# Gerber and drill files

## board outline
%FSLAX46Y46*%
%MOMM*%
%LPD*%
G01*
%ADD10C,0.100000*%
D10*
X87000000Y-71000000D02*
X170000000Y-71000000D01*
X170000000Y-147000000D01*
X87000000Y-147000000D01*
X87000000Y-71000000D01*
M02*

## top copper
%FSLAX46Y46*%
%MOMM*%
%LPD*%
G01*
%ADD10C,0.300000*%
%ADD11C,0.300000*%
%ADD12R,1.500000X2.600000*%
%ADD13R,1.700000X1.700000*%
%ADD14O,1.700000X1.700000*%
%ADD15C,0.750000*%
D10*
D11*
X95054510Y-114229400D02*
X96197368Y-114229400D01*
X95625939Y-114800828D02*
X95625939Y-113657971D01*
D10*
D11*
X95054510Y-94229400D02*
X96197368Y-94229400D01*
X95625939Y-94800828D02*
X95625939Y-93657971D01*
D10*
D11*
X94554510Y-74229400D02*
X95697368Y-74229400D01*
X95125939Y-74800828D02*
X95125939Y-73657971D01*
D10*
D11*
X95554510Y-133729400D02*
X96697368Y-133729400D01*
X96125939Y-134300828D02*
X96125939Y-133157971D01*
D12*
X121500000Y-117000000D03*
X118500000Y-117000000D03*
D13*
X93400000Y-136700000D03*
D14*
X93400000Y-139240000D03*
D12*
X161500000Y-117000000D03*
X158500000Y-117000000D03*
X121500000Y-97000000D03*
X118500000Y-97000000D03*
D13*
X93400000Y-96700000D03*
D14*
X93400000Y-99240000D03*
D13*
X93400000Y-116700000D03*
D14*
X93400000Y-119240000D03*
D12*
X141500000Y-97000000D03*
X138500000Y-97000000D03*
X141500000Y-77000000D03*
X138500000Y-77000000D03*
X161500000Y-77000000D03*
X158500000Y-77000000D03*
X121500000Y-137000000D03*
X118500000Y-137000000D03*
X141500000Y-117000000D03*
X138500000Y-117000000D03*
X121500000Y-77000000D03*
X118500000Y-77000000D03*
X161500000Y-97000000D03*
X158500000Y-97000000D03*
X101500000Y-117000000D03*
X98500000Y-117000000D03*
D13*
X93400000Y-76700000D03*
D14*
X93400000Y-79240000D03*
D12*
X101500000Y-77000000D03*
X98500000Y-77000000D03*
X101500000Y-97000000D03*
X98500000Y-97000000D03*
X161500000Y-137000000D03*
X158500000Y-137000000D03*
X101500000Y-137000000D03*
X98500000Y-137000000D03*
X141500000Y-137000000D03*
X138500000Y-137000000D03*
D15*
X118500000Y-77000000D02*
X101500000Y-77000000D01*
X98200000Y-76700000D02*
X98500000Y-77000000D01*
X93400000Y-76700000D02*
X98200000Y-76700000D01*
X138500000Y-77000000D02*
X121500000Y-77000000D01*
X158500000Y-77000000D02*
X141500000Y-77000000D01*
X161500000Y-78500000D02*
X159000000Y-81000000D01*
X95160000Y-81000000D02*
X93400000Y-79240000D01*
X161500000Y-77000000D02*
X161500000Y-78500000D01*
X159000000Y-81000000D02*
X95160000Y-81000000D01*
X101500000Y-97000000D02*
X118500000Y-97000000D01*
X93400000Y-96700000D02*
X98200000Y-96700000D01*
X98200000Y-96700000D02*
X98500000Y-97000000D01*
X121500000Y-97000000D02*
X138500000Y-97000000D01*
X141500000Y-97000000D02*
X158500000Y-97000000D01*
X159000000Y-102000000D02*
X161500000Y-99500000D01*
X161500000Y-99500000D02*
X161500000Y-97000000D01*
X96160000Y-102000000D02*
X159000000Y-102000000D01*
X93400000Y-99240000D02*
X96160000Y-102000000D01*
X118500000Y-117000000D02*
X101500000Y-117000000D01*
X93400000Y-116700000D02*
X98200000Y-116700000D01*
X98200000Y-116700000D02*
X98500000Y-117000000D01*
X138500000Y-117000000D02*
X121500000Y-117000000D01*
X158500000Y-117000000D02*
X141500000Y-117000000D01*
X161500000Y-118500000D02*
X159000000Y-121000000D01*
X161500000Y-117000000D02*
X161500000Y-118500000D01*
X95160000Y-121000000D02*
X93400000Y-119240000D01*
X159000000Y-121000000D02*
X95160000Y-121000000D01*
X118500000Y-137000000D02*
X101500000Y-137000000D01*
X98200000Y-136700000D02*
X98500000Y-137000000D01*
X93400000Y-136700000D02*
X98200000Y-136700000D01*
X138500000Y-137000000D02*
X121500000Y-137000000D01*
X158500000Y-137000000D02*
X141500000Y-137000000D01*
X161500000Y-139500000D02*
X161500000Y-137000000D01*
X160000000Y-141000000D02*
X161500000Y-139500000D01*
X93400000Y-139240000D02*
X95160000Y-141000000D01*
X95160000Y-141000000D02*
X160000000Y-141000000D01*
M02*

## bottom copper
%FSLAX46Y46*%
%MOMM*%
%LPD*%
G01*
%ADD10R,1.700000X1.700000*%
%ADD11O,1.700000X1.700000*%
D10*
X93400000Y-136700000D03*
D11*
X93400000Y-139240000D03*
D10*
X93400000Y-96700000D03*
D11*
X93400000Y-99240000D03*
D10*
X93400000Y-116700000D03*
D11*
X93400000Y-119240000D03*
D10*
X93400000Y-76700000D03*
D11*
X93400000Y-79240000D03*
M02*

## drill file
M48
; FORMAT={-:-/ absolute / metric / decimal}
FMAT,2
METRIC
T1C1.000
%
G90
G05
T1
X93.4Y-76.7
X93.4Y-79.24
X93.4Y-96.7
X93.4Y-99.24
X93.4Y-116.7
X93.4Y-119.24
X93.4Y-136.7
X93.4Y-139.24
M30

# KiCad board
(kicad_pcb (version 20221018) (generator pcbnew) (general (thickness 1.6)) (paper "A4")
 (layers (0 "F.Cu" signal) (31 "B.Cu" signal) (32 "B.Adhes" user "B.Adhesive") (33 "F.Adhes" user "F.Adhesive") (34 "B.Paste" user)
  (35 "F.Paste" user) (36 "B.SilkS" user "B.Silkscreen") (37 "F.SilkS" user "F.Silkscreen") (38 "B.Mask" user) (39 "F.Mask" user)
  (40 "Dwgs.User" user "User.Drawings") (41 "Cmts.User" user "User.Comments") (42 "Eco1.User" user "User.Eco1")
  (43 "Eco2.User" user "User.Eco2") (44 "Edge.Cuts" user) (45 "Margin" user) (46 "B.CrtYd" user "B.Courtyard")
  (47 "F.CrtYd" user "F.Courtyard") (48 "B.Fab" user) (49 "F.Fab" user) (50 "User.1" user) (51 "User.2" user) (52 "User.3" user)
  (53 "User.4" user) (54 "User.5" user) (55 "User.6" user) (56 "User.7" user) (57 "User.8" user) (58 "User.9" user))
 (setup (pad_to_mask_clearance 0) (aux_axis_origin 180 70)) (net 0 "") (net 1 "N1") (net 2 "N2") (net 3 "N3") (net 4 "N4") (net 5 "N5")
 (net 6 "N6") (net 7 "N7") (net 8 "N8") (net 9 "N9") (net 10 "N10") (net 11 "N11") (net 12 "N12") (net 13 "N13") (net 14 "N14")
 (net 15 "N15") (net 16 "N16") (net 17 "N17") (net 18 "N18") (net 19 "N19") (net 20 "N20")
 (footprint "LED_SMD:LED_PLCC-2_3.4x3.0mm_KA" (layer "F.Cu") (at 120 117 180)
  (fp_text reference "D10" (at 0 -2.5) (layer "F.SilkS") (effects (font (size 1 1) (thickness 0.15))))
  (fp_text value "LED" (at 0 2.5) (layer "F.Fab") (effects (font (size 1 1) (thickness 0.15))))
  (pad "1" smd rect (at -1.5 0 180) (size 1.5 2.6) (layers "F.Cu" "F.Paste" "F.Mask") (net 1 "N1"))
  (pad "2" smd rect (at 1.5 0 180) (size 1.5 2.6) (layers "F.Cu" "F.Paste" "F.Mask") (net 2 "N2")))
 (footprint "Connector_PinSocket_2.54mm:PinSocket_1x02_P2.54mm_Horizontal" (layer "F.Cu") (at 93.4 136.7)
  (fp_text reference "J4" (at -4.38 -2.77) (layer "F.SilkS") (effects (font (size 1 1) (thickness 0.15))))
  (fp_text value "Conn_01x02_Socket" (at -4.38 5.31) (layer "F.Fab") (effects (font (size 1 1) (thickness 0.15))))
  (pad "1" thru_hole rect (at 0 0) (size 1.7 1.7) (drill 1) (layers "*.Cu" "*.Mask") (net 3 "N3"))
  (pad "2" thru_hole oval (at 0 2.54) (size 1.7 1.7) (drill 1) (layers "*.Cu" "*.Mask") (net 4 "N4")))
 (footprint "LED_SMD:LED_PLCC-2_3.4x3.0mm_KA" (layer "F.Cu") (at 160 117 180)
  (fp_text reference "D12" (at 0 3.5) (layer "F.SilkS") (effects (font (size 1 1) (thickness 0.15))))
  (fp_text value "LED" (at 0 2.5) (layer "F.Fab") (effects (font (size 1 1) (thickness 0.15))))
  (pad "1" smd rect (at -1.5 0 180) (size 1.5 2.6) (layers "F.Cu" "F.Paste" "F.Mask") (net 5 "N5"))
  (pad "2" smd rect (at 1.5 0 180) (size 1.5 2.6) (layers "F.Cu" "F.Paste" "F.Mask") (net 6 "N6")))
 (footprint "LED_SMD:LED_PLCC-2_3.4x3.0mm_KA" (layer "F.Cu") (at 120 97 180)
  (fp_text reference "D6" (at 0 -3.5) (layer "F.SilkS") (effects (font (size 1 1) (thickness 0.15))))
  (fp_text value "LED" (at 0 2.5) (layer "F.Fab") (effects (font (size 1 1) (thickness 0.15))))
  (pad "1" smd rect (at -1.5 0 180) (size 1.5 2.6) (layers "F.Cu" "F.Paste" "F.Mask") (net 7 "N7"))
  (pad "2" smd rect (at 1.5 0 180) (size 1.5 2.6) (layers "F.Cu" "F.Paste" "F.Mask") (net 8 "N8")))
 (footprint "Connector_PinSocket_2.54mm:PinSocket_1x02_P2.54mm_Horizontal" (layer "F.Cu") (at 93.4 96.7)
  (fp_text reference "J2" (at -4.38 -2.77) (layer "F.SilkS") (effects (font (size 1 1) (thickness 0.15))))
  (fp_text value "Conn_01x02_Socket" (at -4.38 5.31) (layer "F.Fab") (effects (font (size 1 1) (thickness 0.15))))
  (pad "1" thru_hole rect (at 0 0) (size 1.7 1.7) (drill 1) (layers "*.Cu" "*.Mask") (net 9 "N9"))
  (pad "2" thru_hole oval (at 0 2.54) (size 1.7 1.7) (drill 1) (layers "*.Cu" "*.Mask") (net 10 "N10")))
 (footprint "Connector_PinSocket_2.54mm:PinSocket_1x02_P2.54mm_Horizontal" (layer "F.Cu") (at 93.4 116.7)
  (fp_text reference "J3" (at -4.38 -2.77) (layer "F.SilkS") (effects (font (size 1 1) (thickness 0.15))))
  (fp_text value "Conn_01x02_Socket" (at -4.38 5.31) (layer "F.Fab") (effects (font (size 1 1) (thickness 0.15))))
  (pad "1" thru_hole rect (at 0 0) (size 1.7 1.7) (drill 1) (layers "*.Cu" "*.Mask") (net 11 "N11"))
  (pad "2" thru_hole oval (at 0 2.54) (size 1.7 1.7) (drill 1) (layers "*.Cu" "*.Mask") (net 5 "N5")))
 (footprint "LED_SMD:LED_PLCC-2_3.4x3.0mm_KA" (layer "F.Cu") (at 140 97 180)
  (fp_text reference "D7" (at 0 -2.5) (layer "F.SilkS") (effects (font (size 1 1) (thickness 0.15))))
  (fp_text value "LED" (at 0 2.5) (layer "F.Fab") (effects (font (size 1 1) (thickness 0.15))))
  (pad "1" smd rect (at -1.5 0 180) (size 1.5 2.6) (layers "F.Cu" "F.Paste" "F.Mask") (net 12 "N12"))
  (pad "2" smd rect (at 1.5 0 180) (size 1.5 2.6) (layers "F.Cu" "F.Paste" "F.Mask") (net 7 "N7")))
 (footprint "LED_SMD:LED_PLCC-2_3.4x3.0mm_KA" (layer "F.Cu") (at 140 77 180)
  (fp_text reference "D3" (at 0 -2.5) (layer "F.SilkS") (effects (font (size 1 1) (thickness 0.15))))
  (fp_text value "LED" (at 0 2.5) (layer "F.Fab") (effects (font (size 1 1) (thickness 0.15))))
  (pad "1" smd rect (at -1.5 0 180) (size 1.5 2.6) (layers "F.Cu" "F.Paste" "F.Mask") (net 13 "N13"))
  (pad "2" smd rect (at 1.5 0 180) (size 1.5 2.6) (layers "F.Cu" "F.Paste" "F.Mask") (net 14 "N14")))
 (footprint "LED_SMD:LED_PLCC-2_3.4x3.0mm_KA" (layer "F.Cu") (at 160 77 180)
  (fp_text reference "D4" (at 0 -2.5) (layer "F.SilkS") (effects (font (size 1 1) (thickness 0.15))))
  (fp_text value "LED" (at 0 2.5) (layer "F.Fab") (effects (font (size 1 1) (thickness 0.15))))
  (pad "1" smd rect (at -1.5 0 180) (size 1.5 2.6) (layers "F.Cu" "F.Paste" "F.Mask") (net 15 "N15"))
  (pad "2" smd rect (at 1.5 0 180) (size 1.5 2.6) (layers "F.Cu" "F.Paste" "F.Mask") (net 13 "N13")))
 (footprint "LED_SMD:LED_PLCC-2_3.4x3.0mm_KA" (layer "F.Cu") (at 120 137 180)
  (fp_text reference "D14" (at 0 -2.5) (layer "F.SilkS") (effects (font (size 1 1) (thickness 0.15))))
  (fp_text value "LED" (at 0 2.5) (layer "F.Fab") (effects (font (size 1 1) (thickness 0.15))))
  (pad "1" smd rect (at -1.5 0 180) (size 1.5 2.6) (layers "F.Cu" "F.Paste" "F.Mask") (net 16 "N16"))
  (pad "2" smd rect (at 1.5 0 180) (size 1.5 2.6) (layers "F.Cu" "F.Paste" "F.Mask") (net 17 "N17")))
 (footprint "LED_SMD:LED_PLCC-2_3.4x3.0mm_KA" (layer "F.Cu") (at 140 117 180)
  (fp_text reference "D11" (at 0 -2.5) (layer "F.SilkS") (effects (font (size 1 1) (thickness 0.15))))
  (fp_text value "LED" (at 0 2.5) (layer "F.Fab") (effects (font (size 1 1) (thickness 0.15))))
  (pad "1" smd rect (at -1.5 0 180) (size 1.5 2.6) (layers "F.Cu" "F.Paste" "F.Mask") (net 6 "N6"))
  (pad "2" smd rect (at 1.5 0 180) (size 1.5 2.6) (layers "F.Cu" "F.Paste" "F.Mask") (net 1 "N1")))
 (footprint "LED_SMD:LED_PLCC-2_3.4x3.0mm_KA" (layer "F.Cu") (at 120 77 180)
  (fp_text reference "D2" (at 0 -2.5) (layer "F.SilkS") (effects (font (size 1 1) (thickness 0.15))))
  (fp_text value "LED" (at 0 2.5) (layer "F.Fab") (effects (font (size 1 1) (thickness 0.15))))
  (pad "1" smd rect (at -1.5 0 180) (size 1.5 2.6) (layers "F.Cu" "F.Paste" "F.Mask") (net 14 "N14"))
  (pad "2" smd rect (at 1.5 0 180) (size 1.5 2.6) (layers "F.Cu" "F.Paste" "F.Mask") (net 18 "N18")))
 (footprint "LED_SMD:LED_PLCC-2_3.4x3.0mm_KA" (layer "F.Cu") (at 160 97 180)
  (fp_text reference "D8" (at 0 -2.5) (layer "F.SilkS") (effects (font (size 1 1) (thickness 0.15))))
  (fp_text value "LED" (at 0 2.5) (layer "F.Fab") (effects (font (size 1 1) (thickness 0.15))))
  (pad "1" smd rect (at -1.5 0 180) (size 1.5 2.6) (layers "F.Cu" "F.Paste" "F.Mask") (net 10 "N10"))
  (pad "2" smd rect (at 1.5 0 180) (size 1.5 2.6) (layers "F.Cu" "F.Paste" "F.Mask") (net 12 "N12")))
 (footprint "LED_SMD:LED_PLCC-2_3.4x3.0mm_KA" (layer "F.Cu") (at 100 117 180)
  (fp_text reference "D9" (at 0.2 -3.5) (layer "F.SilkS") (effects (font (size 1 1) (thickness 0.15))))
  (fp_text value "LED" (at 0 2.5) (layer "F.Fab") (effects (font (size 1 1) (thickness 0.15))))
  (pad "1" smd rect (at -1.5 0 180) (size 1.5 2.6) (layers "F.Cu" "F.Paste" "F.Mask") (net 2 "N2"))
  (pad "2" smd rect (at 1.5 0 180) (size 1.5 2.6) (layers "F.Cu" "F.Paste" "F.Mask") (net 11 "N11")))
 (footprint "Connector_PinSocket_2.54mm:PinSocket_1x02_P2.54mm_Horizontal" (layer "F.Cu") (at 93.4 76.7)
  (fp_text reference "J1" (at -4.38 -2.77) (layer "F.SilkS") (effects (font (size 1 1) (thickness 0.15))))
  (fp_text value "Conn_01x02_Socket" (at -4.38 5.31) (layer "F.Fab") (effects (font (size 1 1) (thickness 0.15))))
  (pad "1" thru_hole rect (at 0 0) (size 1.7 1.7) (drill 1) (layers "*.Cu" "*.Mask") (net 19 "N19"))
  (pad "2" thru_hole oval (at 0 2.54) (size 1.7 1.7) (drill 1) (layers "*.Cu" "*.Mask") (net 15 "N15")))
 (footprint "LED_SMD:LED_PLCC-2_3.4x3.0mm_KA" (layer "F.Cu") (at 100 77 180)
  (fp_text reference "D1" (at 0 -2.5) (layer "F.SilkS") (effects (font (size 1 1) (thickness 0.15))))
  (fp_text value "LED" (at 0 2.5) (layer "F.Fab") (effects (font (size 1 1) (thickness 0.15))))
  (pad "1" smd rect (at -1.5 0 180) (size 1.5 2.6) (layers "F.Cu" "F.Paste" "F.Mask") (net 18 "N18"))
  (pad "2" smd rect (at 1.5 0 180) (size 1.5 2.6) (layers "F.Cu" "F.Paste" "F.Mask") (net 19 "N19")))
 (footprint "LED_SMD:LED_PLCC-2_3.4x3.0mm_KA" (layer "F.Cu") (at 100 97 180)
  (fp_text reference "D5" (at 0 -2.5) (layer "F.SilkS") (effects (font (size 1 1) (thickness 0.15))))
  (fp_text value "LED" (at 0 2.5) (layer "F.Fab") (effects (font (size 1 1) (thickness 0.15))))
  (pad "1" smd rect (at -1.5 0 180) (size 1.5 2.6) (layers "F.Cu" "F.Paste" "F.Mask") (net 8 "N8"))
  (pad "2" smd rect (at 1.5 0 180) (size 1.5 2.6) (layers "F.Cu" "F.Paste" "F.Mask") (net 9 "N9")))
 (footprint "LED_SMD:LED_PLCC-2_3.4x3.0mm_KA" (layer "F.Cu") (at 160 137 180)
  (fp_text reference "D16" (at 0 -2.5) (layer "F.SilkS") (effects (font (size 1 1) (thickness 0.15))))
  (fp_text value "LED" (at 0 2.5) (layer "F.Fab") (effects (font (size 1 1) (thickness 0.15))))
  (pad "1" smd rect (at -1.5 0 180) (size 1.5 2.6) (layers "F.Cu" "F.Paste" "F.Mask") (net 4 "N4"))
  (pad "2" smd rect (at 1.5 0 180) (size 1.5 2.6) (layers "F.Cu" "F.Paste" "F.Mask") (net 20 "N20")))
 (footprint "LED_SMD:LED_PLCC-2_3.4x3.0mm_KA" (layer "F.Cu") (at 100 137 180)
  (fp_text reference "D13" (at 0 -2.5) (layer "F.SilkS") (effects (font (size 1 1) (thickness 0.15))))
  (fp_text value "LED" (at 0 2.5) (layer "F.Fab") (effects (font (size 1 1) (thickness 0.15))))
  (pad "1" smd rect (at -1.5 0 180) (size 1.5 2.6) (layers "F.Cu" "F.Paste" "F.Mask") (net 17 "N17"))
  (pad "2" smd rect (at 1.5 0 180) (size 1.5 2.6) (layers "F.Cu" "F.Paste" "F.Mask") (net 3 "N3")))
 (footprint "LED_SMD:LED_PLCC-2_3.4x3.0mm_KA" (layer "F.Cu") (at 140 137 180)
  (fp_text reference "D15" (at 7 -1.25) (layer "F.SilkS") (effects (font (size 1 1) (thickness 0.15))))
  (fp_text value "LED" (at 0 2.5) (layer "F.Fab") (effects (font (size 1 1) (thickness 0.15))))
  (pad "1" smd rect (at -1.5 0 180) (size 1.5 2.6) (layers "F.Cu" "F.Paste" "F.Mask") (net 20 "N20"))
  (pad "2" smd rect (at 1.5 0 180) (size 1.5 2.6) (layers "F.Cu" "F.Paste" "F.Mask") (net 16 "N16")))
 (gr_rect (start 87 71) (end 170 147) (stroke (width 0.1) (type default)) (fill none) (layer "Edge.Cuts"))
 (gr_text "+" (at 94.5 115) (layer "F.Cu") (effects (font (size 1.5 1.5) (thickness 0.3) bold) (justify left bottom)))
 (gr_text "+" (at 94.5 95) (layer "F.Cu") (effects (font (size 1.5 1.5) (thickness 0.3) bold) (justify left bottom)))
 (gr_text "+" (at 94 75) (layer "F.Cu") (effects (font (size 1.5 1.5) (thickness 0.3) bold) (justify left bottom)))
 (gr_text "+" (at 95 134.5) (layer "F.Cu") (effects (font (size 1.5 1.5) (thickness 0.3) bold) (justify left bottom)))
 (segment (start 118.5 77) (end 101.5 77) (width 0.75) (layer "F.Cu") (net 18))
 (segment (start 98.2 76.7) (end 98.5 77) (width 0.75) (layer "F.Cu") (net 19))
 (segment (start 93.4 76.7) (end 98.2 76.7) (width 0.75) (layer "F.Cu") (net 19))
 (segment (start 138.5 77) (end 121.5 77) (width 0.75) (layer "F.Cu") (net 14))
 (segment (start 158.5 77) (end 141.5 77) (width 0.75) (layer "F.Cu") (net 13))
 (segment (start 161.5 78.5) (end 159 81) (width 0.75) (layer "F.Cu") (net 15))
 (segment (start 95.16 81) (end 93.4 79.24) (width 0.75) (layer "F.Cu") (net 15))
 (segment (start 161.5 77) (end 161.5 78.5) (width 0.75) (layer "F.Cu") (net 15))
 (segment (start 159 81) (end 95.16 81) (width 0.75) (layer "F.Cu") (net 15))
 (segment (start 101.5 97) (end 118.5 97) (width 0.75) (layer "F.Cu") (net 8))
 (segment (start 93.4 96.7) (end 98.2 96.7) (width 0.75) (layer "F.Cu") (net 9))
 (segment (start 98.2 96.7) (end 98.5 97) (width 0.75) (layer "F.Cu") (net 9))
 (segment (start 121.5 97) (end 138.5 97) (width 0.75) (layer "F.Cu") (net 7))
 (segment (start 141.5 97) (end 158.5 97) (width 0.75) (layer "F.Cu") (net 12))
 (segment (start 159 102) (end 161.5 99.5) (width 0.75) (layer "F.Cu") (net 10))
 (segment (start 161.5 99.5) (end 161.5 97) (width 0.75) (layer "F.Cu") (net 10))
 (segment (start 96.16 102) (end 159 102) (width 0.75) (layer "F.Cu") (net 10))
 (segment (start 93.4 99.24) (end 96.16 102) (width 0.75) (layer "F.Cu") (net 10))
 (segment (start 118.5 117) (end 101.5 117) (width 0.75) (layer "F.Cu") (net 2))
 (segment (start 93.4 116.7) (end 98.2 116.7) (width 0.75) (layer "F.Cu") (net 11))
 (segment (start 98.2 116.7) (end 98.5 117) (width 0.75) (layer "F.Cu") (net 11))
 (segment (start 138.5 117) (end 121.5 117) (width 0.75) (layer "F.Cu") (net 1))
 (segment (start 158.5 117) (end 141.5 117) (width 0.75) (layer "F.Cu") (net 6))
 (segment (start 161.5 118.5) (end 159 121) (width 0.75) (layer "F.Cu") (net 5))
 (segment (start 161.5 117) (end 161.5 118.5) (width 0.75) (layer "F.Cu") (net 5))
 (segment (start 95.16 121) (end 93.4 119.24) (width 0.75) (layer "F.Cu") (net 5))
 (segment (start 159 121) (end 95.16 121) (width 0.75) (layer "F.Cu") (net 5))
 (segment (start 118.5 137) (end 101.5 137) (width 0.75) (layer "F.Cu") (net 17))
 (segment (start 98.2 136.7) (end 98.5 137) (width 0.75) (layer "F.Cu") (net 3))
 (segment (start 93.4 136.7) (end 98.2 136.7) (width 0.75) (layer "F.Cu") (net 3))
 (segment (start 138.5 137) (end 121.5 137) (width 0.75) (layer "F.Cu") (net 16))
 (segment (start 158.5 137) (end 141.5 137) (width 0.75) (layer "F.Cu") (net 20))
 (segment (start 161.5 139.5) (end 161.5 137) (width 0.75) (layer "F.Cu") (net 4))
 (segment (start 160 141) (end 161.5 139.5) (width 0.75) (layer "F.Cu") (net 4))
 (segment (start 93.4 139.24) (end 95.16 141) (width 0.75) (layer "F.Cu") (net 4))
 (segment (start 95.16 141) (end 160 141) (width 0.75) (layer "F.Cu") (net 4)))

